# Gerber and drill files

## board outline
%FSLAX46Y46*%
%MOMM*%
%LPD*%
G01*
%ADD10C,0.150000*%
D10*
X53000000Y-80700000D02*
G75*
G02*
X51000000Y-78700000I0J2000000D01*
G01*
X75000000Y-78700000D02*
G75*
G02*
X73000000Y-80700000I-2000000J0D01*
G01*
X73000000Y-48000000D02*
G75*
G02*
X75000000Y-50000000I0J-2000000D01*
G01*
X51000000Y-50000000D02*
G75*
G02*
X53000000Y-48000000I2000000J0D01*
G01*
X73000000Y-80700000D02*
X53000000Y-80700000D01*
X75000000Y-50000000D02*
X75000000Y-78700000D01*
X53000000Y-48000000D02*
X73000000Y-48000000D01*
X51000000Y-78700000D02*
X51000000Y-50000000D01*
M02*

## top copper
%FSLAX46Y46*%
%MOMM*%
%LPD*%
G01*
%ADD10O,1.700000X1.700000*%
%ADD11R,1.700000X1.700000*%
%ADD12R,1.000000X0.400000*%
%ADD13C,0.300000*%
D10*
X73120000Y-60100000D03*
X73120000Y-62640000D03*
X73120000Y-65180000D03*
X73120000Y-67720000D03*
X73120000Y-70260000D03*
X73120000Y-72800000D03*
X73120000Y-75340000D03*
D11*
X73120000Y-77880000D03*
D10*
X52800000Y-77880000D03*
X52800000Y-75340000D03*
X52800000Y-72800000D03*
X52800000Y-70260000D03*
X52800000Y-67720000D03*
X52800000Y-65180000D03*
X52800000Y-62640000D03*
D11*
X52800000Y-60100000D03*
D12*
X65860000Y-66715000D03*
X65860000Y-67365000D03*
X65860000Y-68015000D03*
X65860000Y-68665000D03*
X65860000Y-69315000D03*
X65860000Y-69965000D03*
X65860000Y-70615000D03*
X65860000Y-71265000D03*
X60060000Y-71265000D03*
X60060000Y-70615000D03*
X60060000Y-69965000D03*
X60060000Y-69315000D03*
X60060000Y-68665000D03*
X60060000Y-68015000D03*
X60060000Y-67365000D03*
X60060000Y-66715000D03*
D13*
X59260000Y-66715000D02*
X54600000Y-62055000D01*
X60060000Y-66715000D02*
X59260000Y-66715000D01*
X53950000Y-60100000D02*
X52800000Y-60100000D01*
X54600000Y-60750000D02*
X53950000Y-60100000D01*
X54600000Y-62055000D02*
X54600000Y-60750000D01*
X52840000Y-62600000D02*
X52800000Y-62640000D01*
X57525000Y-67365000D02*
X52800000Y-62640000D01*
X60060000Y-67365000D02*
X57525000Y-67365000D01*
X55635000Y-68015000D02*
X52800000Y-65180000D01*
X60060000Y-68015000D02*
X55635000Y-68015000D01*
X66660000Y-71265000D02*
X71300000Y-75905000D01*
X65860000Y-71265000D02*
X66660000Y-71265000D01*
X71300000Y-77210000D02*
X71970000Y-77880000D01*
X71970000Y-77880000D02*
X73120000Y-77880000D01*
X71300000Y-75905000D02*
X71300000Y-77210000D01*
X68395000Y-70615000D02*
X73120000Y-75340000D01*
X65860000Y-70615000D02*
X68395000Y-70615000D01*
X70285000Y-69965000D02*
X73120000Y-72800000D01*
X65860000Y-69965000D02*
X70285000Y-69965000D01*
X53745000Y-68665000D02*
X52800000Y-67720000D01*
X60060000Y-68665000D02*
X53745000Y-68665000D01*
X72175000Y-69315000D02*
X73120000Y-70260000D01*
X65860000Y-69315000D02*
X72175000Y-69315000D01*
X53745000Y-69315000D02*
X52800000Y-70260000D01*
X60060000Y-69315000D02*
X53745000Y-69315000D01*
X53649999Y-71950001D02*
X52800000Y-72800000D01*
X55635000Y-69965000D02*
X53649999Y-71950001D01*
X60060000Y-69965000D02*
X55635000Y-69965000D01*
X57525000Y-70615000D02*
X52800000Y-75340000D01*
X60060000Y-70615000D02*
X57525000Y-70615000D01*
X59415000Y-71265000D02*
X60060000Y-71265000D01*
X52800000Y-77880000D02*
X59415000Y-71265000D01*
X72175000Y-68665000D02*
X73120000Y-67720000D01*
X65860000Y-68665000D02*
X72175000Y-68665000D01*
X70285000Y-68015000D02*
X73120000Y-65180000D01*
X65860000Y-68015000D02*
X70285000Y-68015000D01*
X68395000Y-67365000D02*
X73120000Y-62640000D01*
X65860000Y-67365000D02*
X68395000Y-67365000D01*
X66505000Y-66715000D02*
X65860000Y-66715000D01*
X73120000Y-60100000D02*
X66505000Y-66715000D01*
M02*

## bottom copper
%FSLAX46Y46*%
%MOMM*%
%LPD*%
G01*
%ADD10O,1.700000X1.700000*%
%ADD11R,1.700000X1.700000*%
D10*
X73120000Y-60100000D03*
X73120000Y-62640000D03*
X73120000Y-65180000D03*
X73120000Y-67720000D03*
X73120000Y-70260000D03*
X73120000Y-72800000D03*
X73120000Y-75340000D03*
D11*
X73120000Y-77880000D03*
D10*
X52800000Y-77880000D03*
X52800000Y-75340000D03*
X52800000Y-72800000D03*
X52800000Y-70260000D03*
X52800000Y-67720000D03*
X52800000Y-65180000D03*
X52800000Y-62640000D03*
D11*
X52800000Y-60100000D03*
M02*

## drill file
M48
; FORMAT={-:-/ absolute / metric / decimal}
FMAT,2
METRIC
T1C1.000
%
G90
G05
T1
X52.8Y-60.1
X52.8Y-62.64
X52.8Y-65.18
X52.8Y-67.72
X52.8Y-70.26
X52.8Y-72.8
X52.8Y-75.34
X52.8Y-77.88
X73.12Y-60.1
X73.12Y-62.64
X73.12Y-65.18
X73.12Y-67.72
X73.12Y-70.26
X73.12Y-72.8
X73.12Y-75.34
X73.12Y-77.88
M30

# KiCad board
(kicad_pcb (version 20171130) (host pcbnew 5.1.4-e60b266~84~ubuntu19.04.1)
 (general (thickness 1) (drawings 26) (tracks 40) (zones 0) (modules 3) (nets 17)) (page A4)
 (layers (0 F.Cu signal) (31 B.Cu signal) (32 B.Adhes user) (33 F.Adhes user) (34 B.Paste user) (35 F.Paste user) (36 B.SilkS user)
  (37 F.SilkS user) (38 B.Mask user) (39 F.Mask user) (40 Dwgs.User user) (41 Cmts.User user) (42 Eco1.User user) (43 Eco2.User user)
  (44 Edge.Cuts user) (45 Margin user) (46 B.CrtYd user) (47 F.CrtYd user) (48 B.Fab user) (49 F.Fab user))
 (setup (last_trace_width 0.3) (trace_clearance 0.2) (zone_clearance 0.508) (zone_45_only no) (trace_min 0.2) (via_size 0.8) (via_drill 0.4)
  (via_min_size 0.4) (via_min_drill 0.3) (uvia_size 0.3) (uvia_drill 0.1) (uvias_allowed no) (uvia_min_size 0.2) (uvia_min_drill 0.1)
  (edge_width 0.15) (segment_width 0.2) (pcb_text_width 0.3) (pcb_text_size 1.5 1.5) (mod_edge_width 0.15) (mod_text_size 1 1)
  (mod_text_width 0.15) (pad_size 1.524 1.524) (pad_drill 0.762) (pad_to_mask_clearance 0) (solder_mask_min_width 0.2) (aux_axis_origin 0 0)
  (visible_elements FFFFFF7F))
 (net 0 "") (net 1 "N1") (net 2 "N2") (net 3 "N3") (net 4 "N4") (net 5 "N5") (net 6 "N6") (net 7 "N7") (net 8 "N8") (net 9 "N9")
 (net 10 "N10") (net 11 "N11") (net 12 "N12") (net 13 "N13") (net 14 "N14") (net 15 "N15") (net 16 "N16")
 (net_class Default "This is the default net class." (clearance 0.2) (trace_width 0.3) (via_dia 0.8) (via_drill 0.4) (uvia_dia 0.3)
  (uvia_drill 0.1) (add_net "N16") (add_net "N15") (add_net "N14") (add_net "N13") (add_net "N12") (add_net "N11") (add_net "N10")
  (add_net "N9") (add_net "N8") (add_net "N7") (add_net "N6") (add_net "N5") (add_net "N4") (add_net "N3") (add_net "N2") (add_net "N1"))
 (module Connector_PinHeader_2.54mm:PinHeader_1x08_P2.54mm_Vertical (layer F.Cu) (at 73.12 77.88 180)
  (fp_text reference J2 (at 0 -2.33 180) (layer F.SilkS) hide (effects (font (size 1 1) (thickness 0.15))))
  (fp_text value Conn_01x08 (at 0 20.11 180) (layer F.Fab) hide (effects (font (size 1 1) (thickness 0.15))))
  (pad 8 thru_hole oval (at 0 17.78 180) (size 1.7 1.7) (drill 1) (layers *.Cu *.Mask) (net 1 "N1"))
  (pad 7 thru_hole oval (at 0 15.24 180) (size 1.7 1.7) (drill 1) (layers *.Cu *.Mask) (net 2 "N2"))
  (pad 6 thru_hole oval (at 0 12.7 180) (size 1.7 1.7) (drill 1) (layers *.Cu *.Mask) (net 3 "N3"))
  (pad 5 thru_hole oval (at 0 10.16 180) (size 1.7 1.7) (drill 1) (layers *.Cu *.Mask) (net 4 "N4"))
  (pad 4 thru_hole oval (at 0 7.62 180) (size 1.7 1.7) (drill 1) (layers *.Cu *.Mask) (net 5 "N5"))
  (pad 3 thru_hole oval (at 0 5.08 180) (size 1.7 1.7) (drill 1) (layers *.Cu *.Mask) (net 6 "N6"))
  (pad 2 thru_hole oval (at 0 2.54 180) (size 1.7 1.7) (drill 1) (layers *.Cu *.Mask) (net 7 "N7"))
  (pad 1 thru_hole rect (at 0 0 180) (size 1.7 1.7) (drill 1) (layers *.Cu *.Mask) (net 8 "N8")))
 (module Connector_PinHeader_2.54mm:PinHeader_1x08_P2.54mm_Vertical (layer F.Cu) (at 52.8 60.1)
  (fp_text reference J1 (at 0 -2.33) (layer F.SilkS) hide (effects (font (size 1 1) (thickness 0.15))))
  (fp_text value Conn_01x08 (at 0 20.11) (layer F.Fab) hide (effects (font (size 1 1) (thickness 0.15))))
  (pad 8 thru_hole oval (at 0 17.78) (size 1.7 1.7) (drill 1) (layers *.Cu *.Mask) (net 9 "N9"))
  (pad 7 thru_hole oval (at 0 15.24) (size 1.7 1.7) (drill 1) (layers *.Cu *.Mask) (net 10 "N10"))
  (pad 6 thru_hole oval (at 0 12.7) (size 1.7 1.7) (drill 1) (layers *.Cu *.Mask) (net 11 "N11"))
  (pad 5 thru_hole oval (at 0 10.16) (size 1.7 1.7) (drill 1) (layers *.Cu *.Mask) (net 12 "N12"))
  (pad 4 thru_hole oval (at 0 7.62) (size 1.7 1.7) (drill 1) (layers *.Cu *.Mask) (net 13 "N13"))
  (pad 3 thru_hole oval (at 0 5.08) (size 1.7 1.7) (drill 1) (layers *.Cu *.Mask) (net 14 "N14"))
  (pad 2 thru_hole oval (at 0 2.54) (size 1.7 1.7) (drill 1) (layers *.Cu *.Mask) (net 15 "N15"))
  (pad 1 thru_hole rect (at 0 0) (size 1.7 1.7) (drill 1) (layers *.Cu *.Mask) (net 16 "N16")))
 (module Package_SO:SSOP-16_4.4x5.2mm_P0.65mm (layer F.Cu) (at 62.96 68.99)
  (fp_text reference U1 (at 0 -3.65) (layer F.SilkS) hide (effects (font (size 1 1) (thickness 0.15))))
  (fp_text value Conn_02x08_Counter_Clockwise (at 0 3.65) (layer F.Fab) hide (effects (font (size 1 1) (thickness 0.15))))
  (pad 16 smd rect (at 2.9 -2.275) (size 1 0.4) (layers F.Cu F.Paste F.Mask) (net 1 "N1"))
  (pad 15 smd rect (at 2.9 -1.625) (size 1 0.4) (layers F.Cu F.Paste F.Mask) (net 2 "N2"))
  (pad 14 smd rect (at 2.9 -0.975) (size 1 0.4) (layers F.Cu F.Paste F.Mask) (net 3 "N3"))
  (pad 13 smd rect (at 2.9 -0.325) (size 1 0.4) (layers F.Cu F.Paste F.Mask) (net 4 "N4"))
  (pad 12 smd rect (at 2.9 0.325) (size 1 0.4) (layers F.Cu F.Paste F.Mask) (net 5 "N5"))
  (pad 11 smd rect (at 2.9 0.975) (size 1 0.4) (layers F.Cu F.Paste F.Mask) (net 6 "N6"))
  (pad 10 smd rect (at 2.9 1.625) (size 1 0.4) (layers F.Cu F.Paste F.Mask) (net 7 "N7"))
  (pad 9 smd rect (at 2.9 2.275) (size 1 0.4) (layers F.Cu F.Paste F.Mask) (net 8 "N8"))
  (pad 8 smd rect (at -2.9 2.275) (size 1 0.4) (layers F.Cu F.Paste F.Mask) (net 9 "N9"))
  (pad 7 smd rect (at -2.9 1.625) (size 1 0.4) (layers F.Cu F.Paste F.Mask) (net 10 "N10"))
  (pad 6 smd rect (at -2.9 0.975) (size 1 0.4) (layers F.Cu F.Paste F.Mask) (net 11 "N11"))
  (pad 5 smd rect (at -2.9 0.325) (size 1 0.4) (layers F.Cu F.Paste F.Mask) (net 12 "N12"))
  (pad 4 smd rect (at -2.9 -0.325) (size 1 0.4) (layers F.Cu F.Paste F.Mask) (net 13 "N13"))
  (pad 3 smd rect (at -2.9 -0.975) (size 1 0.4) (layers F.Cu F.Paste F.Mask) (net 14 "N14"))
  (pad 2 smd rect (at -2.9 -1.625) (size 1 0.4) (layers F.Cu F.Paste F.Mask) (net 15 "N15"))
  (pad 1 smd rect (at -2.9 -2.275) (size 1 0.4) (layers F.Cu F.Paste F.Mask) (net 16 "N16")))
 (gr_arc (start 53 78.7) (end 51 78.7) (angle -90) (layer Edge.Cuts) (width 0.15))
 (gr_arc (start 73 78.7) (end 73 80.7) (angle -90) (layer Edge.Cuts) (width 0.15))
 (gr_arc (start 73 50) (end 75 50) (angle -90) (layer Edge.Cuts) (width 0.15))
 (gr_arc (start 53 50) (end 53 48) (angle -90) (layer Edge.Cuts) (width 0.15))
 (gr_line (start 73 80.7) (end 53 80.7) (layer Edge.Cuts) (width 0.15))
 (gr_line (start 75 50) (end 75 78.7) (layer Edge.Cuts) (width 0.15))
 (gr_line (start 53 48) (end 73 48) (layer Edge.Cuts) (width 0.15))
 (gr_line (start 51 78.7) (end 51 50) (layer Edge.Cuts) (width 0.15))
 (segment (start 59.26 66.715) (end 54.6 62.055) (width 0.3) (layer F.Cu) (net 16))
 (segment (start 60.06 66.715) (end 59.26 66.715) (width 0.3) (layer F.Cu) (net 16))
 (segment (start 53.95 60.1) (end 52.8 60.1) (width 0.3) (layer F.Cu) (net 16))
 (segment (start 54.6 60.75) (end 53.95 60.1) (width 0.3) (layer F.Cu) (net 16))
 (segment (start 54.6 62.055) (end 54.6 60.75) (width 0.3) (layer F.Cu) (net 16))
 (segment (start 52.84 62.6) (end 52.8 62.64) (width 0.3) (layer F.Cu) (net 15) (status 30))
 (segment (start 57.525 67.365) (end 52.8 62.64) (width 0.3) (layer F.Cu) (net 15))
 (segment (start 60.06 67.365) (end 57.525 67.365) (width 0.3) (layer F.Cu) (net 15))
 (segment (start 55.635 68.015) (end 52.8 65.18) (width 0.3) (layer F.Cu) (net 14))
 (segment (start 60.06 68.015) (end 55.635 68.015) (width 0.3) (layer F.Cu) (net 14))
 (segment (start 66.66 71.265) (end 71.3 75.905) (width 0.3) (layer F.Cu) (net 8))
 (segment (start 65.86 71.265) (end 66.66 71.265) (width 0.3) (layer F.Cu) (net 8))
 (segment (start 71.3 77.21) (end 71.97 77.88) (width 0.3) (layer F.Cu) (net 8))
 (segment (start 71.97 77.88) (end 73.12 77.88) (width 0.3) (layer F.Cu) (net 8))
 (segment (start 71.3 75.905) (end 71.3 77.21) (width 0.3) (layer F.Cu) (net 8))
 (segment (start 68.395 70.615) (end 73.12 75.34) (width 0.3) (layer F.Cu) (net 7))
 (segment (start 65.86 70.615) (end 68.395 70.615) (width 0.3) (layer F.Cu) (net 7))
 (segment (start 70.285 69.965) (end 73.12 72.8) (width 0.3) (layer F.Cu) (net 6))
 (segment (start 65.86 69.965) (end 70.285 69.965) (width 0.3) (layer F.Cu) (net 6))
 (segment (start 53.745 68.665) (end 52.8 67.72) (width 0.3) (layer F.Cu) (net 13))
 (segment (start 60.06 68.665) (end 53.745 68.665) (width 0.3) (layer F.Cu) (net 13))
 (segment (start 72.175 69.315) (end 73.12 70.26) (width 0.3) (layer F.Cu) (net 5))
 (segment (start 65.86 69.315) (end 72.175 69.315) (width 0.3) (layer F.Cu) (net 5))
 (segment (start 53.745 69.315) (end 52.8 70.26) (width 0.3) (layer F.Cu) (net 12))
 (segment (start 60.06 69.315) (end 53.745 69.315) (width 0.3) (layer F.Cu) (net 12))
 (segment (start 53.649999 71.950001) (end 52.8 72.8) (width 0.3) (layer F.Cu) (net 11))
 (segment (start 55.635 69.965) (end 53.649999 71.950001) (width 0.3) (layer F.Cu) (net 11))
 (segment (start 60.06 69.965) (end 55.635 69.965) (width 0.3) (layer F.Cu) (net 11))
 (segment (start 57.525 70.615) (end 52.8 75.34) (width 0.3) (layer F.Cu) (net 10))
 (segment (start 60.06 70.615) (end 57.525 70.615) (width 0.3) (layer F.Cu) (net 10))
 (segment (start 59.415 71.265) (end 60.06 71.265) (width 0.3) (layer F.Cu) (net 9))
 (segment (start 52.8 77.88) (end 59.415 71.265) (width 0.3) (layer F.Cu) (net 9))
 (segment (start 72.175 68.665) (end 73.12 67.72) (width 0.3) (layer F.Cu) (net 4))
 (segment (start 65.86 68.665) (end 72.175 68.665) (width 0.3) (layer F.Cu) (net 4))
 (segment (start 70.285 68.015) (end 73.12 65.18) (width 0.3) (layer F.Cu) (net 3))
 (segment (start 65.86 68.015) (end 70.285 68.015) (width 0.3) (layer F.Cu) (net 3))
 (segment (start 68.395 67.365) (end 73.12 62.64) (width 0.3) (layer F.Cu) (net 2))
 (segment (start 65.86 67.365) (end 68.395 67.365) (width 0.3) (layer F.Cu) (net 2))
 (segment (start 66.505 66.715) (end 65.86 66.715) (width 0.3) (layer F.Cu) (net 1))
 (segment (start 73.12 60.1) (end 66.505 66.715) (width 0.3) (layer F.Cu) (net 1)))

